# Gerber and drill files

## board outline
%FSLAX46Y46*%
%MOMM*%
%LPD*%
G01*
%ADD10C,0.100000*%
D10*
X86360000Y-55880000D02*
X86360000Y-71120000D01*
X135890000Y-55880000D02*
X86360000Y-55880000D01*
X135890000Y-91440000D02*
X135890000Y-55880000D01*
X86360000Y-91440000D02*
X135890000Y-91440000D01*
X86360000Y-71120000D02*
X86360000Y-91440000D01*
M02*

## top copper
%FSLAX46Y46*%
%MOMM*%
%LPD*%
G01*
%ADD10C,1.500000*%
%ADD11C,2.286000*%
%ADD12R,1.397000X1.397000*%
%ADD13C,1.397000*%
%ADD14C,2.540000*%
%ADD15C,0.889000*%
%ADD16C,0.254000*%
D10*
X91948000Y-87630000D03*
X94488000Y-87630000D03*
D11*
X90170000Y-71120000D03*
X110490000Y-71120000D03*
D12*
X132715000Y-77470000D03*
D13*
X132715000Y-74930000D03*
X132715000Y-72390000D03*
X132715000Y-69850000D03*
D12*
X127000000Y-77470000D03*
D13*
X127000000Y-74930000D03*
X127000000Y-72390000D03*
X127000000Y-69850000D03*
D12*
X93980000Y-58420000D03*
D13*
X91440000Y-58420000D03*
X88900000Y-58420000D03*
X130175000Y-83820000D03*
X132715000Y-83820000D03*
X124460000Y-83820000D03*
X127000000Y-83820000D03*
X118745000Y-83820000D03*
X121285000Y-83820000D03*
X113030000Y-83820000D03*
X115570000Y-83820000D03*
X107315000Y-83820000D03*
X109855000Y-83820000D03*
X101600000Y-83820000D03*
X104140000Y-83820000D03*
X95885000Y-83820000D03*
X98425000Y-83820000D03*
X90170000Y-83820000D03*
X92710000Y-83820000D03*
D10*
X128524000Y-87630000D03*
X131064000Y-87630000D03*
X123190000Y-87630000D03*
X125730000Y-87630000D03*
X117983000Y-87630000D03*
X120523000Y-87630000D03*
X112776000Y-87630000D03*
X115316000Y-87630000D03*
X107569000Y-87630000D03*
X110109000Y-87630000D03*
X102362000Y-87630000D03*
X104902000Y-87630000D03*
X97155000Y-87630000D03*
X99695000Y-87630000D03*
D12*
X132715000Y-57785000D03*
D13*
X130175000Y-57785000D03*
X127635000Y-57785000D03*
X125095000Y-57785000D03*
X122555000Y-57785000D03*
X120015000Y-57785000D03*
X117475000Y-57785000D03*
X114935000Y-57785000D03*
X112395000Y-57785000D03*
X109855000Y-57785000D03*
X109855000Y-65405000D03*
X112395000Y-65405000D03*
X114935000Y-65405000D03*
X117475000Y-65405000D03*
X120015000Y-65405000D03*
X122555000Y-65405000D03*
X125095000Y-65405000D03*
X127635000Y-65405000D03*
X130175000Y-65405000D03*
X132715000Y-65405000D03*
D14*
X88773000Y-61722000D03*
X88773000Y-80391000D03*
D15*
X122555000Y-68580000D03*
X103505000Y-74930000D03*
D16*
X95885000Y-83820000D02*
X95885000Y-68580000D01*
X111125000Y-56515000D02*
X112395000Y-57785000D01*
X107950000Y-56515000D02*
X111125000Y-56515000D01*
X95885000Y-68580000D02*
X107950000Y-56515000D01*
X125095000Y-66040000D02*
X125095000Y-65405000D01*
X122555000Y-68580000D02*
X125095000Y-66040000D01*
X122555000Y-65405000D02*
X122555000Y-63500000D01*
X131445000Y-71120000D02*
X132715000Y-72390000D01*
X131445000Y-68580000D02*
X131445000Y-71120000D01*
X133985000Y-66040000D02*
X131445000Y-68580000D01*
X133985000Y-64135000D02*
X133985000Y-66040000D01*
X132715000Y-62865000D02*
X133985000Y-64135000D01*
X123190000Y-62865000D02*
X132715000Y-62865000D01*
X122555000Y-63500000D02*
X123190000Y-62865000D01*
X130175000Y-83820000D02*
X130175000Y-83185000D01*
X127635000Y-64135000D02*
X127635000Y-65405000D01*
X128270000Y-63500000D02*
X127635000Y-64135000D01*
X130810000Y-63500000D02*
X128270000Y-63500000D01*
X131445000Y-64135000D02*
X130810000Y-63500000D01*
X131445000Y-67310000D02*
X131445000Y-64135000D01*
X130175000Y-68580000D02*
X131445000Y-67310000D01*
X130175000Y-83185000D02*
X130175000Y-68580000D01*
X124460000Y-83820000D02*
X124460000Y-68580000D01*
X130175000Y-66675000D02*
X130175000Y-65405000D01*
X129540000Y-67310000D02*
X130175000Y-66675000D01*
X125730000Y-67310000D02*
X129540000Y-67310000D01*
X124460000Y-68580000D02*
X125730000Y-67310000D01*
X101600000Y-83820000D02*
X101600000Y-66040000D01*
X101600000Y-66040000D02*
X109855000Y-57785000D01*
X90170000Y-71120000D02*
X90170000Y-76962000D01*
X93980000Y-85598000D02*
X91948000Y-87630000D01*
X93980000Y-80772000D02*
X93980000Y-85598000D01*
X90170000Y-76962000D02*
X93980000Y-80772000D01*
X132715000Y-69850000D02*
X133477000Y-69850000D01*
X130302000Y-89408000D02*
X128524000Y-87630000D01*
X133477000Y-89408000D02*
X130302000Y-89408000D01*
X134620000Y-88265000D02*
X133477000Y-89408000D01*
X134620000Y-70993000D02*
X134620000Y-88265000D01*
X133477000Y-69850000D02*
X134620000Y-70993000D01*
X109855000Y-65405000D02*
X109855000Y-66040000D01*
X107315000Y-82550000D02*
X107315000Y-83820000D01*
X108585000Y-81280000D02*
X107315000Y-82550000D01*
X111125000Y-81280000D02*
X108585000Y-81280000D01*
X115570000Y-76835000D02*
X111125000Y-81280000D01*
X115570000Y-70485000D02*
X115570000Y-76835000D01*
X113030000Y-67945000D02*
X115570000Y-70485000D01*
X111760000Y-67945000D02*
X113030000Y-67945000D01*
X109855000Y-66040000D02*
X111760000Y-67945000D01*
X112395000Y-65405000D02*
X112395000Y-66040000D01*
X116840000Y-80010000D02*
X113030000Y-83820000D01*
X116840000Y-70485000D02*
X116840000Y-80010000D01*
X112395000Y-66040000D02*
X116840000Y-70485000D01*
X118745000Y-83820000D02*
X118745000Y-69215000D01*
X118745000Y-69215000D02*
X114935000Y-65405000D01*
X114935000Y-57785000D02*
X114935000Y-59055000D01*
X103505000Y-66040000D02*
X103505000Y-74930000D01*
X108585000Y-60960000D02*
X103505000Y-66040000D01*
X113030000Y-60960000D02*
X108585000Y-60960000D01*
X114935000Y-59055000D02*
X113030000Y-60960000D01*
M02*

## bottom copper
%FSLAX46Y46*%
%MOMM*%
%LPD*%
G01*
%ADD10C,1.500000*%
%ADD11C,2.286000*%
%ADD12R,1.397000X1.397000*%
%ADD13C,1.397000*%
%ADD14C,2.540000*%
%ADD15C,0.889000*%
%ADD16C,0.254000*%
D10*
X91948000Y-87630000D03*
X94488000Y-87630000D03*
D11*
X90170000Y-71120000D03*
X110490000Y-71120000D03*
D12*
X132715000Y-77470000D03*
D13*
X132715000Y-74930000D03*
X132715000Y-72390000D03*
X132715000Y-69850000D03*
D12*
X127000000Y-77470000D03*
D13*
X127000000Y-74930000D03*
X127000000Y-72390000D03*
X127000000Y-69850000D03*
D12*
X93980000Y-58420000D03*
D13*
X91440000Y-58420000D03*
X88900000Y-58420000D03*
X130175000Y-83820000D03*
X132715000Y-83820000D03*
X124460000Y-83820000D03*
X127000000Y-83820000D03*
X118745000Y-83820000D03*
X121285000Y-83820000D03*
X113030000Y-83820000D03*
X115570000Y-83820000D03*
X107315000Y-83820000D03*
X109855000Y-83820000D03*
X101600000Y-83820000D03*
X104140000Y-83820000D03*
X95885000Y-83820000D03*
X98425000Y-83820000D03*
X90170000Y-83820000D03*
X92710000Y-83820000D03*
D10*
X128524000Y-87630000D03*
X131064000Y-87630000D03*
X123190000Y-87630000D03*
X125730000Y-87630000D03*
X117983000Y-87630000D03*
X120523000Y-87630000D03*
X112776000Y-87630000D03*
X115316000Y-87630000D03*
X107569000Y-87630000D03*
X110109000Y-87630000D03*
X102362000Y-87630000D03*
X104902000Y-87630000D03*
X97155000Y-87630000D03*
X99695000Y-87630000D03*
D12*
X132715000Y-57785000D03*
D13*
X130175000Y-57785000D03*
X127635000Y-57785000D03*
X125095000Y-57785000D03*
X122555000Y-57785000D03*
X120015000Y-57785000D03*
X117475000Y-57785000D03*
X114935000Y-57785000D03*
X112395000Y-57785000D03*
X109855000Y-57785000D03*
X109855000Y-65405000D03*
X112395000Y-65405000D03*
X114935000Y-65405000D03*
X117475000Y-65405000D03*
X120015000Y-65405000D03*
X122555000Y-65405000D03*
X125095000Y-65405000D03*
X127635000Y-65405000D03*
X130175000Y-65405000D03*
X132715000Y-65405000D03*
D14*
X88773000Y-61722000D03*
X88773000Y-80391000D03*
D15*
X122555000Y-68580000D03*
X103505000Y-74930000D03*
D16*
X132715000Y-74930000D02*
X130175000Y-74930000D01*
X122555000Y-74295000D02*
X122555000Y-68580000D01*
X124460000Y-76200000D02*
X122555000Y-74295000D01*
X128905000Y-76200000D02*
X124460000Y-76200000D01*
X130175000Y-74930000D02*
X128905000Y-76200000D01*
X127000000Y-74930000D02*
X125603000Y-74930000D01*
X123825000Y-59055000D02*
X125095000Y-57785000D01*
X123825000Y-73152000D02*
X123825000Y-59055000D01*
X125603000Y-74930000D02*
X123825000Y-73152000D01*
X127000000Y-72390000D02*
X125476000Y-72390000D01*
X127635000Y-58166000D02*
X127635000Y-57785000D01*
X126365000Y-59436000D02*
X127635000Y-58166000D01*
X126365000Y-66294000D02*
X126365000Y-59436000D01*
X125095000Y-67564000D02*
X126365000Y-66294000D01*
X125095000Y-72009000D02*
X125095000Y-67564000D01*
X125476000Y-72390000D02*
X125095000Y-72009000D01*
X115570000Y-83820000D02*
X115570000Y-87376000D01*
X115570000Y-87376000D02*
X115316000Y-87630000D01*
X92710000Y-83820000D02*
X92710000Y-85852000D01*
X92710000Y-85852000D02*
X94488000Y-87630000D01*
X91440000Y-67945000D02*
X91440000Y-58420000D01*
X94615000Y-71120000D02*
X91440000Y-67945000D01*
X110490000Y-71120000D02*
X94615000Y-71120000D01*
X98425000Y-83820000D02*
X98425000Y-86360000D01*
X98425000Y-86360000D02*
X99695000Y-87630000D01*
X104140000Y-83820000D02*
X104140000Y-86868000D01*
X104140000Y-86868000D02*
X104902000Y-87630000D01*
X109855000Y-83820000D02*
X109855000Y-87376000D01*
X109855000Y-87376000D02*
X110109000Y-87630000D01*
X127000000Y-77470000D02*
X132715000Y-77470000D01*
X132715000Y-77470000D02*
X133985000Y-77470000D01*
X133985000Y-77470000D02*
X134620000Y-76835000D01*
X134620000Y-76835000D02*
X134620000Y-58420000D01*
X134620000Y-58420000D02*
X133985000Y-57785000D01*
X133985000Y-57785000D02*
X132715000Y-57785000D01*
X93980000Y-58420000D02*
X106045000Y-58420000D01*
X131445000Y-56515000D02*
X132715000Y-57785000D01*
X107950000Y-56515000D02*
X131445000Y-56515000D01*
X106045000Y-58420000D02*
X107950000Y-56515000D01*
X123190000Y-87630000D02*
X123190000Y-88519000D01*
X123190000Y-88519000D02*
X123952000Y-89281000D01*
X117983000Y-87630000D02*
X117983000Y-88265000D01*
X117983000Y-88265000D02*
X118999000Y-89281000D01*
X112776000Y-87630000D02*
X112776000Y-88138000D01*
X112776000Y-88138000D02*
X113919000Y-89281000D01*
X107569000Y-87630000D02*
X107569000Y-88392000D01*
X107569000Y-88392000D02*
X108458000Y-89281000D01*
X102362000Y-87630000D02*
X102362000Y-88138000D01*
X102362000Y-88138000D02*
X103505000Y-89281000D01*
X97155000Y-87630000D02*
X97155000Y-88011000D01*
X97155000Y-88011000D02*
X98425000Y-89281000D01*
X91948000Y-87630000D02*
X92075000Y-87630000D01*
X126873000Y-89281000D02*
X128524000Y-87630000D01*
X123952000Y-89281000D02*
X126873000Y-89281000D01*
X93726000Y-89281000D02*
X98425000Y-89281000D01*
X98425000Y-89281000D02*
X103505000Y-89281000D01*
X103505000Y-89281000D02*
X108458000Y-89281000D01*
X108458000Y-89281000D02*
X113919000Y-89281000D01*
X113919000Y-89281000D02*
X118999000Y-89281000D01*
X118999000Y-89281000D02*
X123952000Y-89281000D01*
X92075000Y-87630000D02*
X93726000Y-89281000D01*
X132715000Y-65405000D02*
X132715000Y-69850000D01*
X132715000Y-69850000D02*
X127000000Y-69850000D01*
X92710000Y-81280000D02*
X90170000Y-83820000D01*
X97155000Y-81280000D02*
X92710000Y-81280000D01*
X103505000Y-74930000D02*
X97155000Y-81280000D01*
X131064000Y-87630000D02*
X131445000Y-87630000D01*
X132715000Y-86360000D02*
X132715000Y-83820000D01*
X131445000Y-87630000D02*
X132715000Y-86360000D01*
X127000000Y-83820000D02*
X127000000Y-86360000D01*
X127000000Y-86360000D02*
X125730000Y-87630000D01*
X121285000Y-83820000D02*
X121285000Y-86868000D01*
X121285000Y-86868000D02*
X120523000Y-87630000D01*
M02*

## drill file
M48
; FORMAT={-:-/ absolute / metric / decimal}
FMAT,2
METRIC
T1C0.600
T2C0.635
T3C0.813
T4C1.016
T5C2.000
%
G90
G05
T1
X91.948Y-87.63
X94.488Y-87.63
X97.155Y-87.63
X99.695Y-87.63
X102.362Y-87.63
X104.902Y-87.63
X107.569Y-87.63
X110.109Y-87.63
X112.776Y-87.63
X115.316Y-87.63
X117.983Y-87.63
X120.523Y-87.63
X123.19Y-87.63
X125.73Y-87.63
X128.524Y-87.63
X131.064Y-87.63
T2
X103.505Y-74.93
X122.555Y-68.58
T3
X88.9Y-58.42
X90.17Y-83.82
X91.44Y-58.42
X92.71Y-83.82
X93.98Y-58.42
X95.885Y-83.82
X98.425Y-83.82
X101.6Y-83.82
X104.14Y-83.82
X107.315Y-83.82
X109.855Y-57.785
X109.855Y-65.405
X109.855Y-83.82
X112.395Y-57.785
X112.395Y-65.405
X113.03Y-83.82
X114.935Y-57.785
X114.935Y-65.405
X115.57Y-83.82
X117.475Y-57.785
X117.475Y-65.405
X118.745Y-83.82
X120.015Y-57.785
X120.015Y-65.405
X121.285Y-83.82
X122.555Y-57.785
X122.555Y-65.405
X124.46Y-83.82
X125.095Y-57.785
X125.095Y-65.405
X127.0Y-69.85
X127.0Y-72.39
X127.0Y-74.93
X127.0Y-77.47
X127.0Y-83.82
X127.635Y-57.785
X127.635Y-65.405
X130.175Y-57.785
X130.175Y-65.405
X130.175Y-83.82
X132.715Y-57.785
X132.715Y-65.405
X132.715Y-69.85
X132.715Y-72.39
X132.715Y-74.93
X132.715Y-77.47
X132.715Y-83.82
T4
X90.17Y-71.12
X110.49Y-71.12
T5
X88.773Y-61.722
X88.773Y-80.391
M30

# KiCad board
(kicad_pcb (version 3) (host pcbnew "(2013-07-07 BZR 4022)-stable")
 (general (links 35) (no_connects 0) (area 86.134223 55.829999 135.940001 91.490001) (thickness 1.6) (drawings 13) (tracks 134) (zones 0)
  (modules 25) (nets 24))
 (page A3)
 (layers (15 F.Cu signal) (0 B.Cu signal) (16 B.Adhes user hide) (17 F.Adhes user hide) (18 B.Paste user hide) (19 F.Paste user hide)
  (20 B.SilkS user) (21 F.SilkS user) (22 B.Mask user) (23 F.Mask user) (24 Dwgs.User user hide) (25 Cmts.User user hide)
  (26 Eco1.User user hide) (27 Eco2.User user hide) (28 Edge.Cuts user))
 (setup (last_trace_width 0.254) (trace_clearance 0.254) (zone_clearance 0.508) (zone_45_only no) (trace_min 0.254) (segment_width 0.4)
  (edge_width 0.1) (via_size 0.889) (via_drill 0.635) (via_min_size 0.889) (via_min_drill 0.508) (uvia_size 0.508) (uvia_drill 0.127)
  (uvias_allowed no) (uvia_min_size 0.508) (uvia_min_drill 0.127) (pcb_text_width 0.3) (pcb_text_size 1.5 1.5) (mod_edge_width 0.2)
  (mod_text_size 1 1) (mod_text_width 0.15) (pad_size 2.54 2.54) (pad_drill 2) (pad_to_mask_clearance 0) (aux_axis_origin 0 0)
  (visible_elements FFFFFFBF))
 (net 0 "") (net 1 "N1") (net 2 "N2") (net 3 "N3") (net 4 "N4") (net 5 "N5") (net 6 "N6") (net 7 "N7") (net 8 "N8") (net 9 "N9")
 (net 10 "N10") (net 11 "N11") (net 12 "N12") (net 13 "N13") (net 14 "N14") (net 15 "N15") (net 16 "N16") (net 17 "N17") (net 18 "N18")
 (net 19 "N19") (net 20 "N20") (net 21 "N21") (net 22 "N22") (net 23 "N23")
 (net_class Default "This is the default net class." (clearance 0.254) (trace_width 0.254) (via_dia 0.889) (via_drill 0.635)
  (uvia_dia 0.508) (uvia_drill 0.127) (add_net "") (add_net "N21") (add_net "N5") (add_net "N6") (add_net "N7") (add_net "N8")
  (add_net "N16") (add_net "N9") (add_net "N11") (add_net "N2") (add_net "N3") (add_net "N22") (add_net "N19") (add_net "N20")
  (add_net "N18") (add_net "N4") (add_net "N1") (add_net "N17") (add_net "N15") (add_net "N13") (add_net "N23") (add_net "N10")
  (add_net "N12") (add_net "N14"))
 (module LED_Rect (layer F.Cu) (at 91.948 87.63)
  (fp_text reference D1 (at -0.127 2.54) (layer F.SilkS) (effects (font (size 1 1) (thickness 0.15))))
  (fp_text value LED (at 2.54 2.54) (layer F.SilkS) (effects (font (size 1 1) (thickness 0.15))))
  (pad 1 thru_hole circle (at 0 0) (size 1.5 1.5) (drill 0.6) (layers *.Cu *.Mask F.SilkS) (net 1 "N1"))
  (pad 2 thru_hole circle (at 2.54 0) (size 1.5 1.5) (drill 0.6) (layers *.Cu *.Mask F.SilkS) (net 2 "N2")))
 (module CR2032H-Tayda (layer F.Cu) (at 97.79 71.12)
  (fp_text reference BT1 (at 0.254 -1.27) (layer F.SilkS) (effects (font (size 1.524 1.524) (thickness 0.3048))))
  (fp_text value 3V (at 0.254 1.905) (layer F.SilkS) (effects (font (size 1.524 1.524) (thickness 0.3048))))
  (pad 2 thru_hole circle (at -7.62 0) (size 2.286 2.286) (drill 1.016) (layers *.Cu *.Mask F.SilkS) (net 1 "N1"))
  (pad 1 thru_hole circle (at 12.7 0) (size 2.286 2.286) (drill 1.016) (layers *.Cu *.Mask F.SilkS) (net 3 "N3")))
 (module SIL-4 (layer F.Cu) (at 132.715 73.66 90)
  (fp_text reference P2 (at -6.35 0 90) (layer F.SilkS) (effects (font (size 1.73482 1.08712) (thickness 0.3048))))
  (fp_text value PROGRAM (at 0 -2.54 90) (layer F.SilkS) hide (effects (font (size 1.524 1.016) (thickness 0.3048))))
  (pad 1 thru_hole rect (at -3.81 0 90) (size 1.397 1.397) (drill 0.8128) (layers *.Cu *.Mask F.SilkS) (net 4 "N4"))
  (pad 2 thru_hole circle (at -1.27 0 90) (size 1.397 1.397) (drill 0.8128) (layers *.Cu *.Mask F.SilkS) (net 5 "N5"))
  (pad 3 thru_hole circle (at 1.27 0 90) (size 1.397 1.397) (drill 0.8128) (layers *.Cu *.Mask F.SilkS) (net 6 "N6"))
  (pad 4 thru_hole circle (at 3.81 0 90) (size 1.397 1.397) (drill 0.8128) (layers *.Cu *.Mask F.SilkS) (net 1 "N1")))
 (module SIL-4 (layer F.Cu) (at 127 73.66 90)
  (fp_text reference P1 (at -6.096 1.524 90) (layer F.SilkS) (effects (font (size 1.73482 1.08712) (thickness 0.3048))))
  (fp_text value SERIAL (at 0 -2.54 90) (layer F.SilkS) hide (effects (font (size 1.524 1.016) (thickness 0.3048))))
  (pad 1 thru_hole rect (at -3.81 0 90) (size 1.397 1.397) (drill 0.8128) (layers *.Cu *.Mask F.SilkS) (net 4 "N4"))
  (pad 2 thru_hole circle (at -1.27 0 90) (size 1.397 1.397) (drill 0.8128) (layers *.Cu *.Mask F.SilkS) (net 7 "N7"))
  (pad 3 thru_hole circle (at 1.27 0 90) (size 1.397 1.397) (drill 0.8128) (layers *.Cu *.Mask F.SilkS) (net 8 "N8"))
  (pad 4 thru_hole circle (at 3.81 0 90) (size 1.397 1.397) (drill 0.8128) (layers *.Cu *.Mask F.SilkS) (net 1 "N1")))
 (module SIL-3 (layer F.Cu) (at 91.44 58.42 180)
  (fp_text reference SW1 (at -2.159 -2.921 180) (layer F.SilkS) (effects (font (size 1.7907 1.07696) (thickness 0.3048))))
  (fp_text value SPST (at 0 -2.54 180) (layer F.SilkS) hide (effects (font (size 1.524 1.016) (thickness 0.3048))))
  (pad 1 thru_hole rect (at -2.54 0 180) (size 1.397 1.397) (drill 0.8128) (layers *.Cu *.Mask F.SilkS) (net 4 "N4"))
  (pad 2 thru_hole circle (at 0 0 180) (size 1.397 1.397) (drill 0.8128) (layers *.Cu *.Mask F.SilkS) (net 3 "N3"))
  (pad 3 thru_hole circle (at 2.54 0 180) (size 1.397 1.397) (drill 0.8128) (layers *.Cu *.Mask F.SilkS)))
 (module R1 (layer F.Cu) (at 131.445 83.82) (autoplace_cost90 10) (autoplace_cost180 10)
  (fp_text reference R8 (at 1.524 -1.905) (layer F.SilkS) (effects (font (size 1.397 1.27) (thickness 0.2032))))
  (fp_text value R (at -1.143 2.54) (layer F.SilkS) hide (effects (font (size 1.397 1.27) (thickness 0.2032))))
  (pad 1 thru_hole circle (at -1.27 0) (size 1.397 1.397) (drill 0.8128) (layers *.Cu *.Mask F.SilkS) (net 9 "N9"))
  (pad 2 thru_hole circle (at 1.27 0) (size 1.397 1.397) (drill 0.8128) (layers *.Cu *.Mask F.SilkS) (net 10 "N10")))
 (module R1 (layer F.Cu) (at 125.73 83.82) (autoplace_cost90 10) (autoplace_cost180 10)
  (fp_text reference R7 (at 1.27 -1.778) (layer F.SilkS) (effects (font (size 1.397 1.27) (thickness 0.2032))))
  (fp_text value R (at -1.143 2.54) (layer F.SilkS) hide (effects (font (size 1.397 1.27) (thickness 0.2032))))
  (pad 1 thru_hole circle (at -1.27 0) (size 1.397 1.397) (drill 0.8128) (layers *.Cu *.Mask F.SilkS) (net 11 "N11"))
  (pad 2 thru_hole circle (at 1.27 0) (size 1.397 1.397) (drill 0.8128) (layers *.Cu *.Mask F.SilkS) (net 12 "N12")))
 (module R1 (layer F.Cu) (at 120.015 83.82) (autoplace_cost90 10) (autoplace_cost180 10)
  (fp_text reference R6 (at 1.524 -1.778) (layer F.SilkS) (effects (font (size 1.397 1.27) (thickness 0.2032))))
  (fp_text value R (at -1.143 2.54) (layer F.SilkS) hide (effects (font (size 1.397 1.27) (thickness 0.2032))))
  (pad 1 thru_hole circle (at -1.27 0) (size 1.397 1.397) (drill 0.8128) (layers *.Cu *.Mask F.SilkS) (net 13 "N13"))
  (pad 2 thru_hole circle (at 1.27 0) (size 1.397 1.397) (drill 0.8128) (layers *.Cu *.Mask F.SilkS) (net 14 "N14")))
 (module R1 (layer F.Cu) (at 114.3 83.82) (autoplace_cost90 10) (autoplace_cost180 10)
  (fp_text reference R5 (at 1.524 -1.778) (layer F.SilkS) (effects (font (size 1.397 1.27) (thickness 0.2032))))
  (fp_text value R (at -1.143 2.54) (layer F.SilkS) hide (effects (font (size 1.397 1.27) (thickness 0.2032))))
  (pad 1 thru_hole circle (at -1.27 0) (size 1.397 1.397) (drill 0.8128) (layers *.Cu *.Mask F.SilkS) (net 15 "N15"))
  (pad 2 thru_hole circle (at 1.27 0) (size 1.397 1.397) (drill 0.8128) (layers *.Cu *.Mask F.SilkS) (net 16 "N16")))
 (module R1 (layer F.Cu) (at 108.585 83.82) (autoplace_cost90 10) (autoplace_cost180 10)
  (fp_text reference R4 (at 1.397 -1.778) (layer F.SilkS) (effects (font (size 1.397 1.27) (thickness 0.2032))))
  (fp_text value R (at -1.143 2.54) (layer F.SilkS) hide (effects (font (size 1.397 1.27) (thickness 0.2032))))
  (pad 1 thru_hole circle (at -1.27 0) (size 1.397 1.397) (drill 0.8128) (layers *.Cu *.Mask F.SilkS) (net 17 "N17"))
  (pad 2 thru_hole circle (at 1.27 0) (size 1.397 1.397) (drill 0.8128) (layers *.Cu *.Mask F.SilkS) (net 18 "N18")))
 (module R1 (layer F.Cu) (at 102.87 83.82) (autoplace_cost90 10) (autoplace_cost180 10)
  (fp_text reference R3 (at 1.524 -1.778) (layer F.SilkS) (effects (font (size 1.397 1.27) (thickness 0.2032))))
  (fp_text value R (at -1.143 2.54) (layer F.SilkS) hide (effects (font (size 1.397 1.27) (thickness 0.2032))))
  (pad 1 thru_hole circle (at -1.27 0) (size 1.397 1.397) (drill 0.8128) (layers *.Cu *.Mask F.SilkS) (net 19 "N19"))
  (pad 2 thru_hole circle (at 1.27 0) (size 1.397 1.397) (drill 0.8128) (layers *.Cu *.Mask F.SilkS) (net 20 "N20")))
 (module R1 (layer F.Cu) (at 97.155 83.82) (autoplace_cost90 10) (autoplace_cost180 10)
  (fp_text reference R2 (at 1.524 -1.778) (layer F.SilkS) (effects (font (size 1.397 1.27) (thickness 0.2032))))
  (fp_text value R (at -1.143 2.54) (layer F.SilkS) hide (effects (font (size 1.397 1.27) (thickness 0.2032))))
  (pad 1 thru_hole circle (at -1.27 0) (size 1.397 1.397) (drill 0.8128) (layers *.Cu *.Mask F.SilkS) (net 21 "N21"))
  (pad 2 thru_hole circle (at 1.27 0) (size 1.397 1.397) (drill 0.8128) (layers *.Cu *.Mask F.SilkS) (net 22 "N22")))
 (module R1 (layer F.Cu) (at 91.44 83.82) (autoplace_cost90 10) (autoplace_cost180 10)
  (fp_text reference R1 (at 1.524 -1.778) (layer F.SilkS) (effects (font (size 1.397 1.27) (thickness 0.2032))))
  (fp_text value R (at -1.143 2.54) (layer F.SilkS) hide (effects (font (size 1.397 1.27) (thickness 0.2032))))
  (pad 1 thru_hole circle (at -1.27 0) (size 1.397 1.397) (drill 0.8128) (layers *.Cu *.Mask F.SilkS) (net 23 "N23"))
  (pad 2 thru_hole circle (at 1.27 0) (size 1.397 1.397) (drill 0.8128) (layers *.Cu *.Mask F.SilkS) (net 2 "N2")))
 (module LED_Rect (layer F.Cu) (at 128.524 87.63)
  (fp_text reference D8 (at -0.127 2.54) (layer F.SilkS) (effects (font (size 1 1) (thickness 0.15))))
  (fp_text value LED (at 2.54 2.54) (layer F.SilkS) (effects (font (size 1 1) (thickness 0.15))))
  (pad 1 thru_hole circle (at 0 0) (size 1.5 1.5) (drill 0.6) (layers *.Cu *.Mask F.SilkS) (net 1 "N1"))
  (pad 2 thru_hole circle (at 2.54 0) (size 1.5 1.5) (drill 0.6) (layers *.Cu *.Mask F.SilkS) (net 10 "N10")))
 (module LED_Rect (layer F.Cu) (at 123.19 87.63)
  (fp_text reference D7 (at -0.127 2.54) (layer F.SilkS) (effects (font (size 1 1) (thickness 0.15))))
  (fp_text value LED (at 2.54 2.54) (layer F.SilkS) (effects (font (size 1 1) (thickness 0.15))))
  (pad 1 thru_hole circle (at 0 0) (size 1.5 1.5) (drill 0.6) (layers *.Cu *.Mask F.SilkS) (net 1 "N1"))
  (pad 2 thru_hole circle (at 2.54 0) (size 1.5 1.5) (drill 0.6) (layers *.Cu *.Mask F.SilkS) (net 12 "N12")))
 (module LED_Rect (layer F.Cu) (at 117.983 87.63)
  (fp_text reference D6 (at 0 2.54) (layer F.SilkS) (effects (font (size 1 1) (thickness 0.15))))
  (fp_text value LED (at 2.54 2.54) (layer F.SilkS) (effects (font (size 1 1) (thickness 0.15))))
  (pad 1 thru_hole circle (at 0 0) (size 1.5 1.5) (drill 0.6) (layers *.Cu *.Mask F.SilkS) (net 1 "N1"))
  (pad 2 thru_hole circle (at 2.54 0) (size 1.5 1.5) (drill 0.6) (layers *.Cu *.Mask F.SilkS) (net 14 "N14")))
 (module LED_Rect (layer F.Cu) (at 112.776 87.63)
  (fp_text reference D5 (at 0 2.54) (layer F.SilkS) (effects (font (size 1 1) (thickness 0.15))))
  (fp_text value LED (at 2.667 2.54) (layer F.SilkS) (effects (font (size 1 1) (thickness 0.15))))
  (pad 1 thru_hole circle (at 0 0) (size 1.5 1.5) (drill 0.6) (layers *.Cu *.Mask F.SilkS) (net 1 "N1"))
  (pad 2 thru_hole circle (at 2.54 0) (size 1.5 1.5) (drill 0.6) (layers *.Cu *.Mask F.SilkS) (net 16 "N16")))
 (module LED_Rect (layer F.Cu) (at 107.569 87.63)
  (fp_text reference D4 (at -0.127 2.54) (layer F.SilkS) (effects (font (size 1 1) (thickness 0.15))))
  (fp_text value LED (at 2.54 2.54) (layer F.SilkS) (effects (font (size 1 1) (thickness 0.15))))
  (pad 1 thru_hole circle (at 0 0) (size 1.5 1.5) (drill 0.6) (layers *.Cu *.Mask F.SilkS) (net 1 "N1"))
  (pad 2 thru_hole circle (at 2.54 0) (size 1.5 1.5) (drill 0.6) (layers *.Cu *.Mask F.SilkS) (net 18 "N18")))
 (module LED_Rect (layer F.Cu) (at 102.362 87.63)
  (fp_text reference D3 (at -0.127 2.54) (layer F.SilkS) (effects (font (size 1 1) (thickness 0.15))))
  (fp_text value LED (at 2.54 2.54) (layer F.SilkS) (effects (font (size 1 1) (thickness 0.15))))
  (pad 1 thru_hole circle (at 0 0) (size 1.5 1.5) (drill 0.6) (layers *.Cu *.Mask F.SilkS) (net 1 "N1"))
  (pad 2 thru_hole circle (at 2.54 0) (size 1.5 1.5) (drill 0.6) (layers *.Cu *.Mask F.SilkS) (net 20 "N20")))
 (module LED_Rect (layer F.Cu) (at 97.155 87.63)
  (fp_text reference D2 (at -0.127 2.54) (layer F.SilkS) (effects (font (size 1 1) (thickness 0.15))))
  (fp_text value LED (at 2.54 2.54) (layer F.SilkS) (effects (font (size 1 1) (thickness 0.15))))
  (pad 1 thru_hole circle (at 0 0) (size 1.5 1.5) (drill 0.6) (layers *.Cu *.Mask F.SilkS) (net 1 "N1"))
  (pad 2 thru_hole circle (at 2.54 0) (size 1.5 1.5) (drill 0.6) (layers *.Cu *.Mask F.SilkS) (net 22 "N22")))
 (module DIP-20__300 (layer F.Cu) (at 121.285 61.595 180)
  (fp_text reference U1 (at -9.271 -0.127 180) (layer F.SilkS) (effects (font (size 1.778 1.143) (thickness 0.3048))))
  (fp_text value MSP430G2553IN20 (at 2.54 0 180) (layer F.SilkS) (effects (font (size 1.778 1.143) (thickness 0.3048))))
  (pad 1 thru_hole rect (at -11.43 3.81 180) (size 1.397 1.397) (drill 0.8128) (layers *.Cu *.Mask F.SilkS) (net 4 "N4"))
  (pad 2 thru_hole circle (at -8.89 3.81 180) (size 1.397 1.397) (drill 0.8128) (layers *.Cu *.Mask F.SilkS))
  (pad 3 thru_hole circle (at -6.35 3.81 180) (size 1.397 1.397) (drill 0.8128) (layers *.Cu *.Mask F.SilkS) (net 8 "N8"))
  (pad 4 thru_hole circle (at -3.81 3.81 180) (size 1.397 1.397) (drill 0.8128) (layers *.Cu *.Mask F.SilkS) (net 7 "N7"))
  (pad 5 thru_hole circle (at -1.27 3.81 180) (size 1.397 1.397) (drill 0.8128) (layers *.Cu *.Mask F.SilkS))
  (pad 6 thru_hole circle (at 1.27 3.81 180) (size 1.397 1.397) (drill 0.8128) (layers *.Cu *.Mask F.SilkS))
  (pad 7 thru_hole circle (at 3.81 3.81 180) (size 1.397 1.397) (drill 0.8128) (layers *.Cu *.Mask F.SilkS))
  (pad 8 thru_hole circle (at 6.35 3.81 180) (size 1.397 1.397) (drill 0.8128) (layers *.Cu *.Mask F.SilkS) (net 23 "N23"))
  (pad 9 thru_hole circle (at 8.89 3.81 180) (size 1.397 1.397) (drill 0.8128) (layers *.Cu *.Mask F.SilkS) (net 21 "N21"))
  (pad 10 thru_hole circle (at 11.43 3.81 180) (size 1.397 1.397) (drill 0.8128) (layers *.Cu *.Mask F.SilkS) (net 19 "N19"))
  (pad 11 thru_hole circle (at 11.43 -3.81 180) (size 1.397 1.397) (drill 0.8128) (layers *.Cu *.Mask F.SilkS) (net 17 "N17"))
  (pad 12 thru_hole circle (at 8.89 -3.81 180) (size 1.397 1.397) (drill 0.8128) (layers *.Cu *.Mask F.SilkS) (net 15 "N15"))
  (pad 13 thru_hole circle (at 6.35 -3.81 180) (size 1.397 1.397) (drill 0.8128) (layers *.Cu *.Mask F.SilkS) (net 13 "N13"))
  (pad 14 thru_hole circle (at 3.81 -3.81 180) (size 1.397 1.397) (drill 0.8128) (layers *.Cu *.Mask F.SilkS))
  (pad 15 thru_hole circle (at 1.27 -3.81 180) (size 1.397 1.397) (drill 0.8128) (layers *.Cu *.Mask F.SilkS))
  (pad 16 thru_hole circle (at -1.27 -3.81 180) (size 1.397 1.397) (drill 0.8128) (layers *.Cu *.Mask F.SilkS) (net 6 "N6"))
  (pad 17 thru_hole circle (at -3.81 -3.81 180) (size 1.397 1.397) (drill 0.8128) (layers *.Cu *.Mask F.SilkS) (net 5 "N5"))
  (pad 18 thru_hole circle (at -6.35 -3.81 180) (size 1.397 1.397) (drill 0.8128) (layers *.Cu *.Mask F.SilkS) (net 9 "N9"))
  (pad 19 thru_hole circle (at -8.89 -3.81 180) (size 1.397 1.397) (drill 0.8128) (layers *.Cu *.Mask F.SilkS) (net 11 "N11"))
  (pad 20 thru_hole circle (at -11.43 -3.81 180) (size 1.397 1.397) (drill 0.8128) (layers *.Cu *.Mask F.SilkS) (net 1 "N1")))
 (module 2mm (layer F.Cu) (at 88.773 61.722)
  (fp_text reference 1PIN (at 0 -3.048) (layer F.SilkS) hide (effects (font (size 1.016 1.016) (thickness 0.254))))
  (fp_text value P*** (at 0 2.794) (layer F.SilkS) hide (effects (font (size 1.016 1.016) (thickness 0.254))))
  (pad "" thru_hole circle (at 0 0) (size 2.54 2.54) (drill 2) (layers *.Cu *.Mask F.SilkS)))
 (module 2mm (layer F.Cu) (at 88.773 80.391)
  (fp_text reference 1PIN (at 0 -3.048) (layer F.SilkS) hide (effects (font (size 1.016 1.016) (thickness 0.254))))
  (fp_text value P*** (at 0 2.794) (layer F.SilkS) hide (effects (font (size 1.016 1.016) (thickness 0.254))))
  (pad "" thru_hole circle (at 0 0) (size 2.54 2.54) (drill 2) (layers *.Cu *.Mask F.SilkS)))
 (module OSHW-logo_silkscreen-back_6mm (layer F.Cu) (at 97.409 65.405)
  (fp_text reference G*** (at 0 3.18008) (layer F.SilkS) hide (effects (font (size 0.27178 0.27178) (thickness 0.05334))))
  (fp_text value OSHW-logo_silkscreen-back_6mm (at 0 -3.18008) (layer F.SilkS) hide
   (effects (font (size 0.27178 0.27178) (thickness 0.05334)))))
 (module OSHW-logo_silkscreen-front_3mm (layer F.Cu) (at 119.38 68.072)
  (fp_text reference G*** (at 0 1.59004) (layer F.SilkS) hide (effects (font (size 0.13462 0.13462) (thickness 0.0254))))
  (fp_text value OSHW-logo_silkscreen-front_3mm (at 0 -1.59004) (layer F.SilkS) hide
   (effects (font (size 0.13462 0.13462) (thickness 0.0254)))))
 (gr_line (start 86.36 55.88) (end 86.36 71.12) (angle 90) (layer Edge.Cuts) (width 0.1))
 (gr_line (start 135.89 55.88) (end 86.36 55.88) (angle 90) (layer Edge.Cuts) (width 0.1))
 (gr_line (start 135.89 91.44) (end 135.89 55.88) (angle 90) (layer Edge.Cuts) (width 0.1))
 (gr_line (start 86.36 91.44) (end 135.89 91.44) (angle 90) (layer Edge.Cuts) (width 0.1))
 (gr_line (start 86.36 71.12) (end 86.36 91.44) (angle 90) (layer Edge.Cuts) (width 0.1))
 (segment (start 95.885 83.82) (end 95.885 68.58) (width 0.254) (layer F.Cu) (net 21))
 (segment (start 111.125 56.515) (end 112.395 57.785) (width 0.254) (layer F.Cu) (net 21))
 (segment (start 107.95 56.515) (end 111.125 56.515) (width 0.254) (layer F.Cu) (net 21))
 (segment (start 95.885 68.58) (end 107.95 56.515) (width 0.254) (layer F.Cu) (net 21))
 (segment (start 132.715 74.93) (end 130.175 74.93) (width 0.254) (layer B.Cu) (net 5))
 (segment (start 125.095 66.04) (end 125.095 65.405) (width 0.254) (layer F.Cu) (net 5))
 (segment (start 122.555 68.58) (end 125.095 66.04) (width 0.254) (layer F.Cu) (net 5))
 (via (at 122.555 68.58) (size 0.889) (layers F.Cu B.Cu) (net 5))
 (segment (start 122.555 74.295) (end 122.555 68.58) (width 0.254) (layer B.Cu) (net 5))
 (segment (start 124.46 76.2) (end 122.555 74.295) (width 0.254) (layer B.Cu) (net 5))
 (segment (start 128.905 76.2) (end 124.46 76.2) (width 0.254) (layer B.Cu) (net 5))
 (segment (start 130.175 74.93) (end 128.905 76.2) (width 0.254) (layer B.Cu) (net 5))
 (segment (start 122.555 65.405) (end 122.555 63.5) (width 0.254) (layer F.Cu) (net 6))
 (segment (start 131.445 71.12) (end 132.715 72.39) (width 0.254) (layer F.Cu) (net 6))
 (segment (start 131.445 68.58) (end 131.445 71.12) (width 0.254) (layer F.Cu) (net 6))
 (segment (start 133.985 66.04) (end 131.445 68.58) (width 0.254) (layer F.Cu) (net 6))
 (segment (start 133.985 64.135) (end 133.985 66.04) (width 0.254) (layer F.Cu) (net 6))
 (segment (start 132.715 62.865) (end 133.985 64.135) (width 0.254) (layer F.Cu) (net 6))
 (segment (start 123.19 62.865) (end 132.715 62.865) (width 0.254) (layer F.Cu) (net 6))
 (segment (start 122.555 63.5) (end 123.19 62.865) (width 0.254) (layer F.Cu) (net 6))
 (segment (start 127 74.93) (end 125.603 74.93) (width 0.254) (layer B.Cu) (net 7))
 (segment (start 123.825 59.055) (end 125.095 57.785) (width 0.254) (layer B.Cu) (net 7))
 (segment (start 123.825 73.152) (end 123.825 59.055) (width 0.254) (layer B.Cu) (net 7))
 (segment (start 125.603 74.93) (end 123.825 73.152) (width 0.254) (layer B.Cu) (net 7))
 (segment (start 127 72.39) (end 125.476 72.39) (width 0.254) (layer B.Cu) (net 8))
 (segment (start 127.635 58.166) (end 127.635 57.785) (width 0.254) (layer B.Cu) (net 8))
 (segment (start 126.365 59.436) (end 127.635 58.166) (width 0.254) (layer B.Cu) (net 8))
 (segment (start 126.365 66.294) (end 126.365 59.436) (width 0.254) (layer B.Cu) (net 8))
 (segment (start 125.095 67.564) (end 126.365 66.294) (width 0.254) (layer B.Cu) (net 8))
 (segment (start 125.095 72.009) (end 125.095 67.564) (width 0.254) (layer B.Cu) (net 8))
 (segment (start 125.476 72.39) (end 125.095 72.009) (width 0.254) (layer B.Cu) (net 8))
 (segment (start 115.57 83.82) (end 115.57 87.376) (width 0.254) (layer B.Cu) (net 16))
 (segment (start 115.57 87.376) (end 115.316 87.63) (width 0.254) (layer B.Cu) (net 16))
 (segment (start 130.175 83.82) (end 130.175 83.185) (width 0.254) (layer F.Cu) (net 9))
 (segment (start 127.635 64.135) (end 127.635 65.405) (width 0.254) (layer F.Cu) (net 9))
 (segment (start 128.27 63.5) (end 127.635 64.135) (width 0.254) (layer F.Cu) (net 9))
 (segment (start 130.81 63.5) (end 128.27 63.5) (width 0.254) (layer F.Cu) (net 9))
 (segment (start 131.445 64.135) (end 130.81 63.5) (width 0.254) (layer F.Cu) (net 9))
 (segment (start 131.445 67.31) (end 131.445 64.135) (width 0.254) (layer F.Cu) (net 9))
 (segment (start 130.175 68.58) (end 131.445 67.31) (width 0.254) (layer F.Cu) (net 9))
 (segment (start 130.175 83.185) (end 130.175 68.58) (width 0.254) (layer F.Cu) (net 9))
 (segment (start 124.46 83.82) (end 124.46 68.58) (width 0.254) (layer F.Cu) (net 11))
 (segment (start 130.175 66.675) (end 130.175 65.405) (width 0.254) (layer F.Cu) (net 11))
 (segment (start 129.54 67.31) (end 130.175 66.675) (width 0.254) (layer F.Cu) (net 11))
 (segment (start 125.73 67.31) (end 129.54 67.31) (width 0.254) (layer F.Cu) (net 11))
 (segment (start 124.46 68.58) (end 125.73 67.31) (width 0.254) (layer F.Cu) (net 11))
 (segment (start 92.71 83.82) (end 92.71 85.852) (width 0.254) (layer B.Cu) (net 2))
 (segment (start 92.71 85.852) (end 94.488 87.63) (width 0.254) (layer B.Cu) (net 2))
 (segment (start 91.44 67.945) (end 91.44 58.42) (width 0.254) (layer B.Cu) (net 3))
 (segment (start 94.615 71.12) (end 91.44 67.945) (width 0.254) (layer B.Cu) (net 3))
 (segment (start 110.49 71.12) (end 94.615 71.12) (width 0.254) (layer B.Cu) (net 3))
 (segment (start 98.425 83.82) (end 98.425 86.36) (width 0.254) (layer B.Cu) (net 22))
 (segment (start 98.425 86.36) (end 99.695 87.63) (width 0.254) (layer B.Cu) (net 22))
 (segment (start 101.6 83.82) (end 101.6 66.04) (width 0.254) (layer F.Cu) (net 19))
 (segment (start 101.6 66.04) (end 109.855 57.785) (width 0.254) (layer F.Cu) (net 19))
 (segment (start 104.14 83.82) (end 104.14 86.868) (width 0.254) (layer B.Cu) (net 20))
 (segment (start 104.14 86.868) (end 104.902 87.63) (width 0.254) (layer B.Cu) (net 20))
 (segment (start 109.855 83.82) (end 109.855 87.376) (width 0.254) (layer B.Cu) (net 18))
 (segment (start 109.855 87.376) (end 110.109 87.63) (width 0.254) (layer B.Cu) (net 18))
 (segment (start 127 77.47) (end 132.715 77.47) (width 0.254) (layer B.Cu) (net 4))
 (segment (start 132.715 77.47) (end 133.985 77.47) (width 0.254) (layer B.Cu) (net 4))
 (segment (start 133.985 77.47) (end 134.62 76.835) (width 0.254) (layer B.Cu) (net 4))
 (segment (start 134.62 76.835) (end 134.62 58.42) (width 0.254) (layer B.Cu) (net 4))
 (segment (start 134.62 58.42) (end 133.985 57.785) (width 0.254) (layer B.Cu) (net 4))
 (segment (start 133.985 57.785) (end 132.715 57.785) (width 0.254) (layer B.Cu) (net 4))
 (segment (start 93.98 58.42) (end 106.045 58.42) (width 0.254) (layer B.Cu) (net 4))
 (segment (start 131.445 56.515) (end 132.715 57.785) (width 0.254) (layer B.Cu) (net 4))
 (segment (start 107.95 56.515) (end 131.445 56.515) (width 0.254) (layer B.Cu) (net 4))
 (segment (start 106.045 58.42) (end 107.95 56.515) (width 0.254) (layer B.Cu) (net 4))
 (segment (start 90.17 71.12) (end 90.17 76.962) (width 0.254) (layer F.Cu) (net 1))
 (segment (start 93.98 85.598) (end 91.948 87.63) (width 0.254) (layer F.Cu) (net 1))
 (segment (start 93.98 80.772) (end 93.98 85.598) (width 0.254) (layer F.Cu) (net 1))
 (segment (start 90.17 76.962) (end 93.98 80.772) (width 0.254) (layer F.Cu) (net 1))
 (segment (start 132.715 69.85) (end 133.477 69.85) (width 0.254) (layer F.Cu) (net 1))
 (segment (start 130.302 89.408) (end 128.524 87.63) (width 0.254) (layer F.Cu) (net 1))
 (segment (start 133.477 89.408) (end 130.302 89.408) (width 0.254) (layer F.Cu) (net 1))
 (segment (start 134.62 88.265) (end 133.477 89.408) (width 0.254) (layer F.Cu) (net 1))
 (segment (start 134.62 70.993) (end 134.62 88.265) (width 0.254) (layer F.Cu) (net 1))
 (segment (start 133.477 69.85) (end 134.62 70.993) (width 0.254) (layer F.Cu) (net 1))
 (segment (start 123.19 87.63) (end 123.19 88.519) (width 0.254) (layer B.Cu) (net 1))
 (segment (start 123.19 88.519) (end 123.952 89.281) (width 0.254) (layer B.Cu) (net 1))
 (segment (start 117.983 87.63) (end 117.983 88.265) (width 0.254) (layer B.Cu) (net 1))
 (segment (start 117.983 88.265) (end 118.999 89.281) (width 0.254) (layer B.Cu) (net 1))
 (segment (start 112.776 87.63) (end 112.776 88.138) (width 0.254) (layer B.Cu) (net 1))
 (segment (start 112.776 88.138) (end 113.919 89.281) (width 0.254) (layer B.Cu) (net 1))
 (segment (start 107.569 87.63) (end 107.569 88.392) (width 0.254) (layer B.Cu) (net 1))
 (segment (start 107.569 88.392) (end 108.458 89.281) (width 0.254) (layer B.Cu) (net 1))
 (segment (start 102.362 87.63) (end 102.362 88.138) (width 0.254) (layer B.Cu) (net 1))
 (segment (start 102.362 88.138) (end 103.505 89.281) (width 0.254) (layer B.Cu) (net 1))
 (segment (start 97.155 87.63) (end 97.155 88.011) (width 0.254) (layer B.Cu) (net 1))
 (segment (start 97.155 88.011) (end 98.425 89.281) (width 0.254) (layer B.Cu) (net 1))
 (segment (start 91.948 87.63) (end 92.075 87.63) (width 0.254) (layer B.Cu) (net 1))
 (segment (start 126.873 89.281) (end 128.524 87.63) (width 0.254) (layer B.Cu) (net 1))
 (segment (start 123.952 89.281) (end 126.873 89.281) (width 0.254) (layer B.Cu) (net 1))
 (segment (start 93.726 89.281) (end 98.425 89.281) (width 0.254) (layer B.Cu) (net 1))
 (segment (start 98.425 89.281) (end 103.505 89.281) (width 0.254) (layer B.Cu) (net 1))
 (segment (start 103.505 89.281) (end 108.458 89.281) (width 0.254) (layer B.Cu) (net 1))
 (segment (start 108.458 89.281) (end 113.919 89.281) (width 0.254) (layer B.Cu) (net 1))
 (segment (start 113.919 89.281) (end 118.999 89.281) (width 0.254) (layer B.Cu) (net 1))
 (segment (start 118.999 89.281) (end 123.952 89.281) (width 0.254) (layer B.Cu) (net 1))
 (segment (start 92.075 87.63) (end 93.726 89.281) (width 0.254) (layer B.Cu) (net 1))
 (segment (start 132.715 65.405) (end 132.715 69.85) (width 0.254) (layer B.Cu) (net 1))
 (segment (start 132.715 69.85) (end 127 69.85) (width 0.254) (layer B.Cu) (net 1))
 (segment (start 109.855 65.405) (end 109.855 66.04) (width 0.254) (layer F.Cu) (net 17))
 (segment (start 107.315 82.55) (end 107.315 83.82) (width 0.254) (layer F.Cu) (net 17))
 (segment (start 108.585 81.28) (end 107.315 82.55) (width 0.254) (layer F.Cu) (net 17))
 (segment (start 111.125 81.28) (end 108.585 81.28) (width 0.254) (layer F.Cu) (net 17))
 (segment (start 115.57 76.835) (end 111.125 81.28) (width 0.254) (layer F.Cu) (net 17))
 (segment (start 115.57 70.485) (end 115.57 76.835) (width 0.254) (layer F.Cu) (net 17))
 (segment (start 113.03 67.945) (end 115.57 70.485) (width 0.254) (layer F.Cu) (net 17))
 (segment (start 111.76 67.945) (end 113.03 67.945) (width 0.254) (layer F.Cu) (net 17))
 (segment (start 109.855 66.04) (end 111.76 67.945) (width 0.254) (layer F.Cu) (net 17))
 (segment (start 112.395 65.405) (end 112.395 66.04) (width 0.254) (layer F.Cu) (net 15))
 (segment (start 116.84 80.01) (end 113.03 83.82) (width 0.254) (layer F.Cu) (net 15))
 (segment (start 116.84 70.485) (end 116.84 80.01) (width 0.254) (layer F.Cu) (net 15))
 (segment (start 112.395 66.04) (end 116.84 70.485) (width 0.254) (layer F.Cu) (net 15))
 (segment (start 118.745 83.82) (end 118.745 69.215) (width 0.254) (layer F.Cu) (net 13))
 (segment (start 118.745 69.215) (end 114.935 65.405) (width 0.254) (layer F.Cu) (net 13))
 (segment (start 114.935 57.785) (end 114.935 59.055) (width 0.254) (layer F.Cu) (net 23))
 (segment (start 92.71 81.28) (end 90.17 83.82) (width 0.254) (layer B.Cu) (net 23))
 (segment (start 97.155 81.28) (end 92.71 81.28) (width 0.254) (layer B.Cu) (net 23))
 (segment (start 103.505 74.93) (end 97.155 81.28) (width 0.254) (layer B.Cu) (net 23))
 (via (at 103.505 74.93) (size 0.889) (layers F.Cu B.Cu) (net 23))
 (segment (start 103.505 66.04) (end 103.505 74.93) (width 0.254) (layer F.Cu) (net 23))
 (segment (start 108.585 60.96) (end 103.505 66.04) (width 0.254) (layer F.Cu) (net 23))
 (segment (start 113.03 60.96) (end 108.585 60.96) (width 0.254) (layer F.Cu) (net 23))
 (segment (start 114.935 59.055) (end 113.03 60.96) (width 0.254) (layer F.Cu) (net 23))
 (segment (start 131.064 87.63) (end 131.445 87.63) (width 0.254) (layer B.Cu) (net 10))
 (segment (start 132.715 86.36) (end 132.715 83.82) (width 0.254) (layer B.Cu) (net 10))
 (segment (start 131.445 87.63) (end 132.715 86.36) (width 0.254) (layer B.Cu) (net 10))
 (segment (start 127 83.82) (end 127 86.36) (width 0.254) (layer B.Cu) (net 12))
 (segment (start 127 86.36) (end 125.73 87.63) (width 0.254) (layer B.Cu) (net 12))
 (segment (start 121.285 83.82) (end 121.285 86.868) (width 0.254) (layer B.Cu) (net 14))
 (segment (start 121.285 86.868) (end 120.523 87.63) (width 0.254) (layer B.Cu) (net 14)))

